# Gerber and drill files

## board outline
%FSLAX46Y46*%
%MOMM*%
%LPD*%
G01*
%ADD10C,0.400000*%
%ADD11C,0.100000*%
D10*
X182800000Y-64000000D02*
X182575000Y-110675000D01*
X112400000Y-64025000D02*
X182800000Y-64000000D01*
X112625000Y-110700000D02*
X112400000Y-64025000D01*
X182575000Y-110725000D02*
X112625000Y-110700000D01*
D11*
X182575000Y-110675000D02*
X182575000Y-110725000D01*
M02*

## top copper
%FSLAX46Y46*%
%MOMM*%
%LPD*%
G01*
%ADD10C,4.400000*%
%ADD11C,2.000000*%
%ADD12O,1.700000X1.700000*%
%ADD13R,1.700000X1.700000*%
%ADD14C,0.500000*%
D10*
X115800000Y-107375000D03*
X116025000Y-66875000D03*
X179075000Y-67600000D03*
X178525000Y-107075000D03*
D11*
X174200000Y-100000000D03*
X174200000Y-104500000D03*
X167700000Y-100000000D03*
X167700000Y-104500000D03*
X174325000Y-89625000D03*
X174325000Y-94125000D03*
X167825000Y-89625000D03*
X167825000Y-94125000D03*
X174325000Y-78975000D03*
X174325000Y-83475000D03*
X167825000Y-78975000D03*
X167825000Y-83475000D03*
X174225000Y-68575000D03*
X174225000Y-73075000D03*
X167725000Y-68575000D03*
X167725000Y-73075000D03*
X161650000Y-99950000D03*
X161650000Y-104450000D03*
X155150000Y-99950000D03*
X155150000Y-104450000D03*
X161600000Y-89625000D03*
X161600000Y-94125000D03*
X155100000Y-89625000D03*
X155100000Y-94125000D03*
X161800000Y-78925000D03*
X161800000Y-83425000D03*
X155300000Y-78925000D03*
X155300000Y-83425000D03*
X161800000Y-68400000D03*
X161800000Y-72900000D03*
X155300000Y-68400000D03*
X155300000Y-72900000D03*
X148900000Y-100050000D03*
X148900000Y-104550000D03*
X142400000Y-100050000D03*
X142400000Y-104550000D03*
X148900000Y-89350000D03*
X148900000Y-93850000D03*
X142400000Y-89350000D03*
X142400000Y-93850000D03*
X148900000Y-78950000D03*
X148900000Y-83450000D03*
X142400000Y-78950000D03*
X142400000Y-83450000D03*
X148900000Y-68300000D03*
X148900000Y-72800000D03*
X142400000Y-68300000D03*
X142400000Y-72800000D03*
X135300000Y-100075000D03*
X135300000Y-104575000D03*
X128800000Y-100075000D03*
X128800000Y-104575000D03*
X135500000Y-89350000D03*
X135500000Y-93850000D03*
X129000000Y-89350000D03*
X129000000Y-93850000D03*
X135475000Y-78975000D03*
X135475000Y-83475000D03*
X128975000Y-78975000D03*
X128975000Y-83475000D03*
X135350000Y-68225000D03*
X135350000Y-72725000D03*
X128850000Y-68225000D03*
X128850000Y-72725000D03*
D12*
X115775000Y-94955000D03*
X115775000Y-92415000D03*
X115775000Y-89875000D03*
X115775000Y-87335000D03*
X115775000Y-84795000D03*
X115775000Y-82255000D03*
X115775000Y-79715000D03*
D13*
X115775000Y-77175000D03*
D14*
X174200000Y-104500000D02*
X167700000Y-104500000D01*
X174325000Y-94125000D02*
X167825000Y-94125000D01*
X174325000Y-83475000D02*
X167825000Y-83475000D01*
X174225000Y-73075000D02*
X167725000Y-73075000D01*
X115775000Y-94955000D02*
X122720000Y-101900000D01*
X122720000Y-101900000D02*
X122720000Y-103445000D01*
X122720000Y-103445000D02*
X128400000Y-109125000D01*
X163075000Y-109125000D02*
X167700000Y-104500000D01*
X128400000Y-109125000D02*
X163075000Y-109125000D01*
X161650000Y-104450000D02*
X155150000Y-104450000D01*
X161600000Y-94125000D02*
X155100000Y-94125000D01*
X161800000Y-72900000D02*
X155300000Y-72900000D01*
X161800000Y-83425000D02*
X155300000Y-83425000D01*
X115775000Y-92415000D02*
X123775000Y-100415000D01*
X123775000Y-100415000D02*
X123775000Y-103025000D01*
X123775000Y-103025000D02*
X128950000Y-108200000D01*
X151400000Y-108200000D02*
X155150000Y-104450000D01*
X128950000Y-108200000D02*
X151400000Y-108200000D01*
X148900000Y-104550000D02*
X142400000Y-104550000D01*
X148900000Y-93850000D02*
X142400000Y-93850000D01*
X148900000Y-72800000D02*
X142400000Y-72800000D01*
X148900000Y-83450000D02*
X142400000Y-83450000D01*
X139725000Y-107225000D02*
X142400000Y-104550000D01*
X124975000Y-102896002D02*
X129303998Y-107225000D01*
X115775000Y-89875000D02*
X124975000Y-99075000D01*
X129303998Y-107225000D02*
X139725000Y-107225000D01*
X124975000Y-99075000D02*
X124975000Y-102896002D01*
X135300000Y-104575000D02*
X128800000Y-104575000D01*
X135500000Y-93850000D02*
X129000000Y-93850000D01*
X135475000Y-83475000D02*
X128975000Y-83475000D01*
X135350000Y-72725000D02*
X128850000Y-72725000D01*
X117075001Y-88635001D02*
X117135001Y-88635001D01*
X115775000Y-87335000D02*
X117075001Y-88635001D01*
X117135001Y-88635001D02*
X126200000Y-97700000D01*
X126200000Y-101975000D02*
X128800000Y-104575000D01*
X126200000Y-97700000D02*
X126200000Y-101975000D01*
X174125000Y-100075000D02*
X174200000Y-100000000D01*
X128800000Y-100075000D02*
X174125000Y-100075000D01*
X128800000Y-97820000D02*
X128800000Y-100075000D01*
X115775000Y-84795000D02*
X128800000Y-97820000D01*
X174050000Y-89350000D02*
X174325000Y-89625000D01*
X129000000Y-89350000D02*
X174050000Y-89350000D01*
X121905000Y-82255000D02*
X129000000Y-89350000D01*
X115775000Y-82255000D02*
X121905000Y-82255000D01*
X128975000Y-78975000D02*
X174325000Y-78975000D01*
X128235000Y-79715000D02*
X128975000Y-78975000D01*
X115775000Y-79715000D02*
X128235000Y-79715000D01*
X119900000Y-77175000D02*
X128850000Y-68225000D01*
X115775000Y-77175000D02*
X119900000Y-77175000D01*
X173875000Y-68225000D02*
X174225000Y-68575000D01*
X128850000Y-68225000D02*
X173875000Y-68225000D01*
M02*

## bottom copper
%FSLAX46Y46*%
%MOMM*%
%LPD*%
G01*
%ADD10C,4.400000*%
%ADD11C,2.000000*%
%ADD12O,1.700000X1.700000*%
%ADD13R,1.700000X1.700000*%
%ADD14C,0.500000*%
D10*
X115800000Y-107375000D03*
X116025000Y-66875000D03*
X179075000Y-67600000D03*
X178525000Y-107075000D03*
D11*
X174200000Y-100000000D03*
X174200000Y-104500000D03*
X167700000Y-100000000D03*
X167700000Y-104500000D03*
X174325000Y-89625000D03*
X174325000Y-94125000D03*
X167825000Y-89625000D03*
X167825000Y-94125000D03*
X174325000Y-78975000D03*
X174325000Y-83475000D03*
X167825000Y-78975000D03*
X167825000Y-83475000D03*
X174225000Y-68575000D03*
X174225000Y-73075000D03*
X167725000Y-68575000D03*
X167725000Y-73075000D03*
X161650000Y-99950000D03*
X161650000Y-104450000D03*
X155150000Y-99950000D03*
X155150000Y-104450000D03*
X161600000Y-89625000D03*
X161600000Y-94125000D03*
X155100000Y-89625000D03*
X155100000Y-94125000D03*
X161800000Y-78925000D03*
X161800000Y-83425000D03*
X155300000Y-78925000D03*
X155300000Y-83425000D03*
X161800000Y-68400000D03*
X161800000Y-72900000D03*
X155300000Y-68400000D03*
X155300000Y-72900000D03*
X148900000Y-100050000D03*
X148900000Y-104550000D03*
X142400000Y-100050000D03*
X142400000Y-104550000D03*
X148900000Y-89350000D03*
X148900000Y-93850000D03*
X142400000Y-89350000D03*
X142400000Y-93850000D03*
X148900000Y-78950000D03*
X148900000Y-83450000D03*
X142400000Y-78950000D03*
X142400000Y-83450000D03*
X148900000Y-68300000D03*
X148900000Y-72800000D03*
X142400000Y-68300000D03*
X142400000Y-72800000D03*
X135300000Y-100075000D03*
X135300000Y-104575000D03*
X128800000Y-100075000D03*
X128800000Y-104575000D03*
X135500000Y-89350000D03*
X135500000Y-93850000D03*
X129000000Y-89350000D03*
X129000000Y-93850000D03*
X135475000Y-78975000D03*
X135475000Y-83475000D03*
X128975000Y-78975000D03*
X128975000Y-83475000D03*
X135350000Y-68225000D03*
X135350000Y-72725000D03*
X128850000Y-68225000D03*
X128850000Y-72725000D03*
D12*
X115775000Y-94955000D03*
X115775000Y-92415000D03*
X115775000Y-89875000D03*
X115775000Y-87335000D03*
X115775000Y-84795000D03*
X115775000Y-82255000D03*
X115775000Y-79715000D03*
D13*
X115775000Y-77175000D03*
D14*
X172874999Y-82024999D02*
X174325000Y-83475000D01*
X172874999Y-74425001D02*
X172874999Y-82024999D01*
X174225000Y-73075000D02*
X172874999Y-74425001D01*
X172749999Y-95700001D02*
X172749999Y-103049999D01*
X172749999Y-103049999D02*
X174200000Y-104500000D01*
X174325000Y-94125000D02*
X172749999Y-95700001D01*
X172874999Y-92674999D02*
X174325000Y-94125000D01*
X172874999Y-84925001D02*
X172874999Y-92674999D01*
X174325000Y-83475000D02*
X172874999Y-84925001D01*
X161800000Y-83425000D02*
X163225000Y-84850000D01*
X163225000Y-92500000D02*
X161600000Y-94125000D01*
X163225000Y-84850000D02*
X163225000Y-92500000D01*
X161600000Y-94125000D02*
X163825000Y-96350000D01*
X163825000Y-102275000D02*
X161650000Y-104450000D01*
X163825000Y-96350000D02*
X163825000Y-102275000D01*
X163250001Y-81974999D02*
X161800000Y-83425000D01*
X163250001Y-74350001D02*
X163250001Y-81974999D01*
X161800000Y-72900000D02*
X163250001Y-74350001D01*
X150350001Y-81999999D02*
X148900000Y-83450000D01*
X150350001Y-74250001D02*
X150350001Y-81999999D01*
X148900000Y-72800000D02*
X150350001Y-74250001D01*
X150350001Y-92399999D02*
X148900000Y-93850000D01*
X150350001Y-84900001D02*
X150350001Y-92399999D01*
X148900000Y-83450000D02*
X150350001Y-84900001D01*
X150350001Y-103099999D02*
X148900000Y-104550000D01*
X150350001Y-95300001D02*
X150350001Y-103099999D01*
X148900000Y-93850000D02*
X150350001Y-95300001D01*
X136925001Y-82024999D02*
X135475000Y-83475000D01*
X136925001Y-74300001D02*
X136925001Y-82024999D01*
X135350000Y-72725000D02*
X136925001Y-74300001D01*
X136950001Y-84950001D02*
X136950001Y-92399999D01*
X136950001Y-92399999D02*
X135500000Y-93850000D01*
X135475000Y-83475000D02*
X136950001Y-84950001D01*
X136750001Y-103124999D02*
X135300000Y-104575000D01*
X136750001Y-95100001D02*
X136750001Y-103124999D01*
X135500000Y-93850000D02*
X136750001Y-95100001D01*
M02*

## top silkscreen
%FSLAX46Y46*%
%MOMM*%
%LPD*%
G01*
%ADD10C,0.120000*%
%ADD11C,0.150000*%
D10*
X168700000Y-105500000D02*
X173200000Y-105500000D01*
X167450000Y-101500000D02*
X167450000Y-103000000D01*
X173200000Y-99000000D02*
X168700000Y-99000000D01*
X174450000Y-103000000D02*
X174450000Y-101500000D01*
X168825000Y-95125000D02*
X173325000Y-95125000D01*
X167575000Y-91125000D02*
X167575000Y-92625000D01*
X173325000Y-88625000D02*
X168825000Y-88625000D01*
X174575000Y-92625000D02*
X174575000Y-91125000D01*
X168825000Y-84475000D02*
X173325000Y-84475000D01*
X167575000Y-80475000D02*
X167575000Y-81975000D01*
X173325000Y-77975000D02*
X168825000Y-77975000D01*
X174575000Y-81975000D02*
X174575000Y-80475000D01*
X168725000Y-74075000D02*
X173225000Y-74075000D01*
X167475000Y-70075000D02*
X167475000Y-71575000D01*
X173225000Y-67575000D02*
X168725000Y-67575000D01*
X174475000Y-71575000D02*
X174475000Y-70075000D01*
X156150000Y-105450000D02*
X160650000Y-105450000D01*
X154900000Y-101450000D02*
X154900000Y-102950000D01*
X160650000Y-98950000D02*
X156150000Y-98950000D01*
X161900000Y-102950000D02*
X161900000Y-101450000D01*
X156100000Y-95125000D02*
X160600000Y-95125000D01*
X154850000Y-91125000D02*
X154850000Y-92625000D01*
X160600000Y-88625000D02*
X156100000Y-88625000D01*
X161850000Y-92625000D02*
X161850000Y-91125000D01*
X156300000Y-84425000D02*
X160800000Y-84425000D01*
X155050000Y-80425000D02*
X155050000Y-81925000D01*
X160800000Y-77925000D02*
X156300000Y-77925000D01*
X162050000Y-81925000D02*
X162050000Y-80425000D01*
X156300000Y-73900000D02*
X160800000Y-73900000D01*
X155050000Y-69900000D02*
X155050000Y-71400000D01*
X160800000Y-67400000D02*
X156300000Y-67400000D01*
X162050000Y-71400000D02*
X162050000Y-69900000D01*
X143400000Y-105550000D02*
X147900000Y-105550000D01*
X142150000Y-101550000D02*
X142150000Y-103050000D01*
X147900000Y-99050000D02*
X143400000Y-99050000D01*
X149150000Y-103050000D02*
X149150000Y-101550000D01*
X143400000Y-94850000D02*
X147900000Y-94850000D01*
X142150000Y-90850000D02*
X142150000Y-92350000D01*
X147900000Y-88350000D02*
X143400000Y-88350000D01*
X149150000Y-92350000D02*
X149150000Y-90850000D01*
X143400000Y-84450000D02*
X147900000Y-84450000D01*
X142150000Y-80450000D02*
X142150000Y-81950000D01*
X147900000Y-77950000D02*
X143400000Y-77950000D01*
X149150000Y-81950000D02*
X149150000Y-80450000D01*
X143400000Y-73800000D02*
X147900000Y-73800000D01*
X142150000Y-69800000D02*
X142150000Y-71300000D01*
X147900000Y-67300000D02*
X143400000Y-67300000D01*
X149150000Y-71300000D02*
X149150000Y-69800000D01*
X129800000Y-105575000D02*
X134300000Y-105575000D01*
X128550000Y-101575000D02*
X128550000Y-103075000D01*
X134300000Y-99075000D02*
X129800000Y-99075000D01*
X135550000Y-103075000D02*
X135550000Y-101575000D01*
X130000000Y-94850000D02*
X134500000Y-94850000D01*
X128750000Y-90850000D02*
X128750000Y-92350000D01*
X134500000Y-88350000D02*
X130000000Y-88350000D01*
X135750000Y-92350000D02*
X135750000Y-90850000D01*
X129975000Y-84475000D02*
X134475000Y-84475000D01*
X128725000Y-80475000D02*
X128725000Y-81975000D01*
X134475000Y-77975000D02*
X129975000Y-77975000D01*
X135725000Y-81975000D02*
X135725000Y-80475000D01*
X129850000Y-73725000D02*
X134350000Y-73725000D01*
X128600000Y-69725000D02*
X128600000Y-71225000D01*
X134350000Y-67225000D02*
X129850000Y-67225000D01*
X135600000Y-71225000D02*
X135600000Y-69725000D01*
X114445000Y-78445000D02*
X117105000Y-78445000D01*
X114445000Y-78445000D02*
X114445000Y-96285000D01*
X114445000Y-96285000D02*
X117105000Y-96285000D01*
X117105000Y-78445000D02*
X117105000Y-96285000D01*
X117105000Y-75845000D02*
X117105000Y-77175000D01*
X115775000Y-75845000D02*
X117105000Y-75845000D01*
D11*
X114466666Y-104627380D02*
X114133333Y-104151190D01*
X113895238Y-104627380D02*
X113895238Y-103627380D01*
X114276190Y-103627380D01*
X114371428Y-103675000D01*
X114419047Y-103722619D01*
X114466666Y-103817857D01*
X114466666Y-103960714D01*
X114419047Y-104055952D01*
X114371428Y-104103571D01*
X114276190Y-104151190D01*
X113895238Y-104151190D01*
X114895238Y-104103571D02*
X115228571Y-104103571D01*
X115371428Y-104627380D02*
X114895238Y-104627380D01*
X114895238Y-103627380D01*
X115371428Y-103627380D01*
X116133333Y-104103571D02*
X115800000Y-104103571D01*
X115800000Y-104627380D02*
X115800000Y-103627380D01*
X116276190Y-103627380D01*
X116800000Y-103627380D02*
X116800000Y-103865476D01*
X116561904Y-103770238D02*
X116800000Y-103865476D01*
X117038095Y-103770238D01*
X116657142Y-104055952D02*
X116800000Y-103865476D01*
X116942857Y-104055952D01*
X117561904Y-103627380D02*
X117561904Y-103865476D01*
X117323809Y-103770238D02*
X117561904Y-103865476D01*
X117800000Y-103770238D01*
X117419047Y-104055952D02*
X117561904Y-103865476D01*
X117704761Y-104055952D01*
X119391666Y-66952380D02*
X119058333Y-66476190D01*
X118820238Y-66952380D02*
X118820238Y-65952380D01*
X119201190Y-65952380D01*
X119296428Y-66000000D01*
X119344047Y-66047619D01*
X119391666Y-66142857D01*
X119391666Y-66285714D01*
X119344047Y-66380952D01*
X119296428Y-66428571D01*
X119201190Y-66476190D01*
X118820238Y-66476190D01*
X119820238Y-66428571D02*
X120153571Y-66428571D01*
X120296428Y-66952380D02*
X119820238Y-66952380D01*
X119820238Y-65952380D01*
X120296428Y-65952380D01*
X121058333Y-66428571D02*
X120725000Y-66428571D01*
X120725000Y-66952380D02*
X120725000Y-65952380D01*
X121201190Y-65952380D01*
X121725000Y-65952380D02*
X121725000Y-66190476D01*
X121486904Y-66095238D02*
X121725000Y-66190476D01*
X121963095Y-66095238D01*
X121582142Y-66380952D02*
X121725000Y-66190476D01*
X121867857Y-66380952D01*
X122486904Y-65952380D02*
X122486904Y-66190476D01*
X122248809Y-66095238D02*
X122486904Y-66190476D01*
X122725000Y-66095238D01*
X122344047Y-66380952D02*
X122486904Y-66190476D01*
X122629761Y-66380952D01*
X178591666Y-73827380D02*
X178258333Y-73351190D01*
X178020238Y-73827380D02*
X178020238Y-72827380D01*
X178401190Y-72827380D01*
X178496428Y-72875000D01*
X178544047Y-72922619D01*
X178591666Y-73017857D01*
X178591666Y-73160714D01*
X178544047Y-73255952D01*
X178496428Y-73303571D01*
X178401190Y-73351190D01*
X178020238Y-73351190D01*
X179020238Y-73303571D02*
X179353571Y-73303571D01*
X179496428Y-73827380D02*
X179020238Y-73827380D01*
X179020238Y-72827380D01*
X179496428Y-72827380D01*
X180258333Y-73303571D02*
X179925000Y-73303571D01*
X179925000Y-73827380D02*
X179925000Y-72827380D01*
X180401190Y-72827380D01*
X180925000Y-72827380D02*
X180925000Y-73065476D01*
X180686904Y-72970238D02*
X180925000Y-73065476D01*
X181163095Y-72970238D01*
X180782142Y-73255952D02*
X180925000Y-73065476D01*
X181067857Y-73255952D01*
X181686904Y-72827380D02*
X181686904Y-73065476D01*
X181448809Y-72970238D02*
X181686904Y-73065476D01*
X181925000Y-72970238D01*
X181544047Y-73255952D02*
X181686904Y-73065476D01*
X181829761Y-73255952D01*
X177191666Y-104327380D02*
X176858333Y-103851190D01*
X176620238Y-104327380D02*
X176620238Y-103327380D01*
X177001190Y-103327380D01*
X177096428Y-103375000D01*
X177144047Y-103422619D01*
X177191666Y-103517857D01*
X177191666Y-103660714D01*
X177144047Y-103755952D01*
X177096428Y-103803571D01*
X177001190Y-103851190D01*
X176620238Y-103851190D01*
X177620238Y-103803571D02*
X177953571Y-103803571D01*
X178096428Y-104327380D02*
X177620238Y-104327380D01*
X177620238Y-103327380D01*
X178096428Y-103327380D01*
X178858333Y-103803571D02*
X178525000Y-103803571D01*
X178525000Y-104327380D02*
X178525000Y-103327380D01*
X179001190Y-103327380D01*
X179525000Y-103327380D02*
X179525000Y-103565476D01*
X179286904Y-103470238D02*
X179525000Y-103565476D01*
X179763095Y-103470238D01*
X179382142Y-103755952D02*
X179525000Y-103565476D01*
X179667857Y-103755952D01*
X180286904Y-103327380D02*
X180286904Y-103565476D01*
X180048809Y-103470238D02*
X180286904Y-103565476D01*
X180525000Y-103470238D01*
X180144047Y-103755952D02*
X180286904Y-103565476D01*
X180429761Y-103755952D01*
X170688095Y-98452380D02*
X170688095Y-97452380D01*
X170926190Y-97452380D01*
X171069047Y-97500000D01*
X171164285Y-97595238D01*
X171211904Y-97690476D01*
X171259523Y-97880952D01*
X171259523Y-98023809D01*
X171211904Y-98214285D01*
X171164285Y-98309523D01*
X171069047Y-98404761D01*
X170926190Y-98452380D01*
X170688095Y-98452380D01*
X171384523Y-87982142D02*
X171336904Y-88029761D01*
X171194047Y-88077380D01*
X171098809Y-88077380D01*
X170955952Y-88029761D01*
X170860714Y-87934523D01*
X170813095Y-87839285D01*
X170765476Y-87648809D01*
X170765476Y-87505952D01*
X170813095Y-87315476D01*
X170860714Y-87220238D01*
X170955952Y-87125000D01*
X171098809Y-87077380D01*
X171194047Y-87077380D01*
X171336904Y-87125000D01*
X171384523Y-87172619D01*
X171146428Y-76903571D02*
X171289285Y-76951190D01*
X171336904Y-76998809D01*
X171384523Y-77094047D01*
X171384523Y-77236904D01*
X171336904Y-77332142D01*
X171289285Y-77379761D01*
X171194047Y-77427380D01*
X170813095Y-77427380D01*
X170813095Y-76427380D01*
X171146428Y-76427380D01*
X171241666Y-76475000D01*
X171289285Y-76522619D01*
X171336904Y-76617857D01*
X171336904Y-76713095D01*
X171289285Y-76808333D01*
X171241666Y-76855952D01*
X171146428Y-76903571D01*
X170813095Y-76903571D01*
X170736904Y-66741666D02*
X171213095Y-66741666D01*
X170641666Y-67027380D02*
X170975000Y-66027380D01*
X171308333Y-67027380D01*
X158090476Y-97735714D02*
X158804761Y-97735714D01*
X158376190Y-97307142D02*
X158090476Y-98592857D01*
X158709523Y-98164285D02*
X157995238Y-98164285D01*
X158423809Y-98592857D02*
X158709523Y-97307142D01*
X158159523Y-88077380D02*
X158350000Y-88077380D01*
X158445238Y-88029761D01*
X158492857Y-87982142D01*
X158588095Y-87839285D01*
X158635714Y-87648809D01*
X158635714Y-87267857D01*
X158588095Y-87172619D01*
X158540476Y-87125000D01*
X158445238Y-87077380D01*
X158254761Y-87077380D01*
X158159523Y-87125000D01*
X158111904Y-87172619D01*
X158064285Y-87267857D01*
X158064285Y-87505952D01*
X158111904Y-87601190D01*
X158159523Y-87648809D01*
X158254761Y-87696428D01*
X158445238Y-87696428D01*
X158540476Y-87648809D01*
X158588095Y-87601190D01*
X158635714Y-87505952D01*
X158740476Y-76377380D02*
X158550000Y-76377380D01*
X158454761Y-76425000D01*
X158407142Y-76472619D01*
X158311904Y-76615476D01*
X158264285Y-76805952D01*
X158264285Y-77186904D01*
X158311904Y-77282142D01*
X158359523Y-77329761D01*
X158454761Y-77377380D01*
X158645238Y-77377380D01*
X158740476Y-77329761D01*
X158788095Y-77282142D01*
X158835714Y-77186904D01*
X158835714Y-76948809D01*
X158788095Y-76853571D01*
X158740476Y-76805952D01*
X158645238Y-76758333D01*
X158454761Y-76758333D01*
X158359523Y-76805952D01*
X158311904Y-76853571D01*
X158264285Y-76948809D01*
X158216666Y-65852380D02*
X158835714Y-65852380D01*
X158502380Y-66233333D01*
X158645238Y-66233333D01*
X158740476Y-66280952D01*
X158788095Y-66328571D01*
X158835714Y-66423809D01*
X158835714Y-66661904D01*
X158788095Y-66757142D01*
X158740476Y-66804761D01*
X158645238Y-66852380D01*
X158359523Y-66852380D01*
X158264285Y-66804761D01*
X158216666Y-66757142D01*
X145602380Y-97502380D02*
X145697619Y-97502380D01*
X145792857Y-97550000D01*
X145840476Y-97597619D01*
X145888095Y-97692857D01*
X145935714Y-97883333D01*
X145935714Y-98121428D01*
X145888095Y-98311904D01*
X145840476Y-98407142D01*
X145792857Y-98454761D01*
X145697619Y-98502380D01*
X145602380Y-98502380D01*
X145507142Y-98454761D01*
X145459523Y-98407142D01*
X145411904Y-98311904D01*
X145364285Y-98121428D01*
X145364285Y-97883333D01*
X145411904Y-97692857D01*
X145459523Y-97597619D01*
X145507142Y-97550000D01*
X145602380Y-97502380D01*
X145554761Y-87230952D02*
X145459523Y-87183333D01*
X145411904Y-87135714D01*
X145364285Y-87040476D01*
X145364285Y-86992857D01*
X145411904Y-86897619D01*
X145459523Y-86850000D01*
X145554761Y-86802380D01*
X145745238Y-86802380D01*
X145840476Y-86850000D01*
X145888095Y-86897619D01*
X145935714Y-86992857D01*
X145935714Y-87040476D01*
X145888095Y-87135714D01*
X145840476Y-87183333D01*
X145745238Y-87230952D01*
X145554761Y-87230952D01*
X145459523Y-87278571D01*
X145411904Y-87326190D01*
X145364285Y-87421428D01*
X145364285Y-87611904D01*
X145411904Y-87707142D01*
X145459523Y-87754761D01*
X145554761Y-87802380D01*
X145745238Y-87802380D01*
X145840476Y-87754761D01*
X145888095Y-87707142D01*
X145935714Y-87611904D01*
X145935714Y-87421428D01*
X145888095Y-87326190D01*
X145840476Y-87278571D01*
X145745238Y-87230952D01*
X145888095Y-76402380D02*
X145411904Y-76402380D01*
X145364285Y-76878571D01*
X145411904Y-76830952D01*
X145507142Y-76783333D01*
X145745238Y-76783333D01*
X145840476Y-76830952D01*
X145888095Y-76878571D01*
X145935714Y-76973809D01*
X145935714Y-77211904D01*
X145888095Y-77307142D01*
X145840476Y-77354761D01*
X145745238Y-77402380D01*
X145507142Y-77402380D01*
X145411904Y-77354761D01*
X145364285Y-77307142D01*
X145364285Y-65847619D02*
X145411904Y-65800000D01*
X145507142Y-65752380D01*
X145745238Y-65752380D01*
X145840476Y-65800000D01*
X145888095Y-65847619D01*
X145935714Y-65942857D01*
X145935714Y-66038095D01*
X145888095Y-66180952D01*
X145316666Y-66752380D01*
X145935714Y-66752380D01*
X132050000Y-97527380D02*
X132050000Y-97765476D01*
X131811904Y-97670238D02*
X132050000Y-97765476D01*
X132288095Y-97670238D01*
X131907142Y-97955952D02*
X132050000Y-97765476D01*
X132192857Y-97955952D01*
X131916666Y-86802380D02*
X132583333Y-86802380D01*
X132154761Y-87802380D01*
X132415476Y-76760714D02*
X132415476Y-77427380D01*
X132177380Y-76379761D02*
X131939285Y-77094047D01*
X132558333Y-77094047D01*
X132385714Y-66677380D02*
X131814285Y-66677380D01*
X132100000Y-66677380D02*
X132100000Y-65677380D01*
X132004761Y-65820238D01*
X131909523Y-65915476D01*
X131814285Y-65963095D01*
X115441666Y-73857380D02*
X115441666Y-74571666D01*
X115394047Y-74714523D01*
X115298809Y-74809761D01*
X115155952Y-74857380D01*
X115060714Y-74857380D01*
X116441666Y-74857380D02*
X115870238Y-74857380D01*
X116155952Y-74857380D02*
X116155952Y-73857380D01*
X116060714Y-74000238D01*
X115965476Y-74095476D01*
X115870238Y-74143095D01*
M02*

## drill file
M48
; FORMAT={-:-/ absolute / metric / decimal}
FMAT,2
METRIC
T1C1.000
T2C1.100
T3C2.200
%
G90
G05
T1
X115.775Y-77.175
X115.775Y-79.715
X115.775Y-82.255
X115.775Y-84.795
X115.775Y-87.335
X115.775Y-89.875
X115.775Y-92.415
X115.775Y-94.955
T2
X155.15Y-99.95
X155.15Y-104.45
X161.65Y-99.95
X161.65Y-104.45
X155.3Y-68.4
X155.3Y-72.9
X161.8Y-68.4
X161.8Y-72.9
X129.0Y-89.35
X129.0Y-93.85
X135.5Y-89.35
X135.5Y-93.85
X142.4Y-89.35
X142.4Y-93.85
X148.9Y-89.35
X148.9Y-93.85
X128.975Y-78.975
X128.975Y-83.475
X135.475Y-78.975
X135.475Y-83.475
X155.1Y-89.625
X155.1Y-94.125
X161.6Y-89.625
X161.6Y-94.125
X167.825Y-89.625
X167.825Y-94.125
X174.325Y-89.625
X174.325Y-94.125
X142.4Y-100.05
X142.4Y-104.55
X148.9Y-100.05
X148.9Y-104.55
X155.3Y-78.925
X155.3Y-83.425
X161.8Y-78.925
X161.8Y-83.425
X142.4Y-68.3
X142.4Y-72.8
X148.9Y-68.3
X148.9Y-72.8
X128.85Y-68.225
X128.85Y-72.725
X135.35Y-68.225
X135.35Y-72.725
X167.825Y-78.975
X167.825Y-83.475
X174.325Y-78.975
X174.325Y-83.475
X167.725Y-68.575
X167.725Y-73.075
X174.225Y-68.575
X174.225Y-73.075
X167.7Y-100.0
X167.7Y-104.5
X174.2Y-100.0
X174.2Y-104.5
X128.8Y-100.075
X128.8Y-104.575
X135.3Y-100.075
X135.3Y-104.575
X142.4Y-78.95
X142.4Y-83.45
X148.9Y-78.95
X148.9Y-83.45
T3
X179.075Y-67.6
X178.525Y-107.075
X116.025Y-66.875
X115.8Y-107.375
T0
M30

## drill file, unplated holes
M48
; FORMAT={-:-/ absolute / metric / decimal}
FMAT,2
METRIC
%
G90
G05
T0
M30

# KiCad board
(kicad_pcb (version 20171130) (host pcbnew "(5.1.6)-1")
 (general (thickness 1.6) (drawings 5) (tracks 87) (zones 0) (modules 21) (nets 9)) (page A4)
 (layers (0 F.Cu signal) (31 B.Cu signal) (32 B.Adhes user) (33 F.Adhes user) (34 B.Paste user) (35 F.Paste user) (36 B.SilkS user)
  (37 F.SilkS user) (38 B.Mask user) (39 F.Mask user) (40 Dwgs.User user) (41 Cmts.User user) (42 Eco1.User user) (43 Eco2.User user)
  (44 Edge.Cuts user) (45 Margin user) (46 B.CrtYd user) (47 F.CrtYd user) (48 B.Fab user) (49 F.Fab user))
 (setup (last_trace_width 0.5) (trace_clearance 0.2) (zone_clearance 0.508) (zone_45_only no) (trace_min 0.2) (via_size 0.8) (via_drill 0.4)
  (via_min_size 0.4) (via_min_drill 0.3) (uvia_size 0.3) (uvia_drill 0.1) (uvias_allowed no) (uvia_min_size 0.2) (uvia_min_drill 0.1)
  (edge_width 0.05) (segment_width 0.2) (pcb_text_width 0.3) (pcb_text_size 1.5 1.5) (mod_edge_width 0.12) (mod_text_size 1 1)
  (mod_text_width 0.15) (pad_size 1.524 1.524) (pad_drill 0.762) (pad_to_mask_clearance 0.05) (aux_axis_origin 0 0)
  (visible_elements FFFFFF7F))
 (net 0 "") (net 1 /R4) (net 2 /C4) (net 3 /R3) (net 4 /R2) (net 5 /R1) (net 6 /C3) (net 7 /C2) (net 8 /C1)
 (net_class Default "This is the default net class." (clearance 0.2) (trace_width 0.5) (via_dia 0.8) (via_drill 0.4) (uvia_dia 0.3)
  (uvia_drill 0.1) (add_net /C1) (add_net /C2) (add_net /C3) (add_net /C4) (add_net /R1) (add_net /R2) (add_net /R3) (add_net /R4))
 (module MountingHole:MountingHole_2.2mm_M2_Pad (layer F.Cu) (at 115.8 107.375)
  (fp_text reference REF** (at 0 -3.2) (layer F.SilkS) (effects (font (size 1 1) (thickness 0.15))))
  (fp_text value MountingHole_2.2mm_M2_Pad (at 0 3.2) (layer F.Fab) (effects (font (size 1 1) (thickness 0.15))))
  (pad 1 thru_hole circle (at 0 0) (size 4.4 4.4) (drill 2.2) (layers *.Cu *.Mask)))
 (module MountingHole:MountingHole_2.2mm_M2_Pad (layer F.Cu) (at 116.025 66.875)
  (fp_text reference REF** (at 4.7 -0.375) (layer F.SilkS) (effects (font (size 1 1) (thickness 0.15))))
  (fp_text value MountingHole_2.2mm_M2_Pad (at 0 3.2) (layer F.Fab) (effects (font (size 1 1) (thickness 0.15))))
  (pad 1 thru_hole circle (at 0 0) (size 4.4 4.4) (drill 2.2) (layers *.Cu *.Mask)))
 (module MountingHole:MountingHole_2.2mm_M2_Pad (layer F.Cu) (at 179.075 67.6)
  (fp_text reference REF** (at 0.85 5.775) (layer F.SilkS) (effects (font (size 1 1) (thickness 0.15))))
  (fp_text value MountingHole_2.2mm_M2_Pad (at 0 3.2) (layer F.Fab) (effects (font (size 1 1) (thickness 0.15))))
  (pad 1 thru_hole circle (at 0 0) (size 4.4 4.4) (drill 2.2) (layers *.Cu *.Mask)))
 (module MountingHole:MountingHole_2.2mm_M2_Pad (layer F.Cu) (at 178.525 107.075)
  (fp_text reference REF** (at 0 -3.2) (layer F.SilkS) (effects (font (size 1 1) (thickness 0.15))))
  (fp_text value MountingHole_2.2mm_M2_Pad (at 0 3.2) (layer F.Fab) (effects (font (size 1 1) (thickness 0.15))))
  (pad 1 thru_hole circle (at 0 0) (size 4.4 4.4) (drill 2.2) (layers *.Cu *.Mask)))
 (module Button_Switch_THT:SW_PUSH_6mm (layer F.Cu) (at 167.7 100)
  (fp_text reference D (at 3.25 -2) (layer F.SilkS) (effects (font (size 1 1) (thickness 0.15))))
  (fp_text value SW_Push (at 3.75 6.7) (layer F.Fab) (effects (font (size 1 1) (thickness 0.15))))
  (fp_line (start 1 5.5) (end 5.5 5.5) (layer F.SilkS) (width 0.12))
  (fp_line (start -0.25 1.5) (end -0.25 3) (layer F.SilkS) (width 0.12))
  (fp_line (start 5.5 -1) (end 1 -1) (layer F.SilkS) (width 0.12))
  (fp_line (start 6.75 3) (end 6.75 1.5) (layer F.SilkS) (width 0.12))
  (pad 1 thru_hole circle (at 6.5 0 90) (size 2 2) (drill 1.1) (layers *.Cu *.Mask) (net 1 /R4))
  (pad 2 thru_hole circle (at 6.5 4.5 90) (size 2 2) (drill 1.1) (layers *.Cu *.Mask) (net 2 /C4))
  (pad 1 thru_hole circle (at 0 0 90) (size 2 2) (drill 1.1) (layers *.Cu *.Mask) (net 1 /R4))
  (pad 2 thru_hole circle (at 0 4.5 90) (size 2 2) (drill 1.1) (layers *.Cu *.Mask) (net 2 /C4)))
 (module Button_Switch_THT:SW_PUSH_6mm (layer F.Cu) (at 167.825 89.625)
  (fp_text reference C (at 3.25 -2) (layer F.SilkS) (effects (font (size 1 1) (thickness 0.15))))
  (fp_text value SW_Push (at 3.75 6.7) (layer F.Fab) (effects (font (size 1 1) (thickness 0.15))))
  (fp_line (start 1 5.5) (end 5.5 5.5) (layer F.SilkS) (width 0.12))
  (fp_line (start -0.25 1.5) (end -0.25 3) (layer F.SilkS) (width 0.12))
  (fp_line (start 5.5 -1) (end 1 -1) (layer F.SilkS) (width 0.12))
  (fp_line (start 6.75 3) (end 6.75 1.5) (layer F.SilkS) (width 0.12))
  (pad 1 thru_hole circle (at 6.5 0 90) (size 2 2) (drill 1.1) (layers *.Cu *.Mask) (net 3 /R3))
  (pad 2 thru_hole circle (at 6.5 4.5 90) (size 2 2) (drill 1.1) (layers *.Cu *.Mask) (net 2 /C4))
  (pad 1 thru_hole circle (at 0 0 90) (size 2 2) (drill 1.1) (layers *.Cu *.Mask) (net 3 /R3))
  (pad 2 thru_hole circle (at 0 4.5 90) (size 2 2) (drill 1.1) (layers *.Cu *.Mask) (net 2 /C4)))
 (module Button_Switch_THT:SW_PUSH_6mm (layer F.Cu) (at 167.825 78.975)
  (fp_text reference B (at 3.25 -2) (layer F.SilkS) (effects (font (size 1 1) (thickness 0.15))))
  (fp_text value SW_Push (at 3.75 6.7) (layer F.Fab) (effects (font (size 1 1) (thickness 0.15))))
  (fp_line (start 1 5.5) (end 5.5 5.5) (layer F.SilkS) (width 0.12))
  (fp_line (start -0.25 1.5) (end -0.25 3) (layer F.SilkS) (width 0.12))
  (fp_line (start 5.5 -1) (end 1 -1) (layer F.SilkS) (width 0.12))
  (fp_line (start 6.75 3) (end 6.75 1.5) (layer F.SilkS) (width 0.12))
  (pad 1 thru_hole circle (at 6.5 0 90) (size 2 2) (drill 1.1) (layers *.Cu *.Mask) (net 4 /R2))
  (pad 2 thru_hole circle (at 6.5 4.5 90) (size 2 2) (drill 1.1) (layers *.Cu *.Mask) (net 2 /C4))
  (pad 1 thru_hole circle (at 0 0 90) (size 2 2) (drill 1.1) (layers *.Cu *.Mask) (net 4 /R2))
  (pad 2 thru_hole circle (at 0 4.5 90) (size 2 2) (drill 1.1) (layers *.Cu *.Mask) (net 2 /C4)))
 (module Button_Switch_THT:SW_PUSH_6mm (layer F.Cu) (at 167.725 68.575)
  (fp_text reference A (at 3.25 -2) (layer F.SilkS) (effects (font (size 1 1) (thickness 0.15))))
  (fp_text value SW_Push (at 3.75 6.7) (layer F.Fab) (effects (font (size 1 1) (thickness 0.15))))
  (fp_line (start 1 5.5) (end 5.5 5.5) (layer F.SilkS) (width 0.12))
  (fp_line (start -0.25 1.5) (end -0.25 3) (layer F.SilkS) (width 0.12))
  (fp_line (start 5.5 -1) (end 1 -1) (layer F.SilkS) (width 0.12))
  (fp_line (start 6.75 3) (end 6.75 1.5) (layer F.SilkS) (width 0.12))
  (pad 1 thru_hole circle (at 6.5 0 90) (size 2 2) (drill 1.1) (layers *.Cu *.Mask) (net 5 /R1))
  (pad 2 thru_hole circle (at 6.5 4.5 90) (size 2 2) (drill 1.1) (layers *.Cu *.Mask) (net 2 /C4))
  (pad 1 thru_hole circle (at 0 0 90) (size 2 2) (drill 1.1) (layers *.Cu *.Mask) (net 5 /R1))
  (pad 2 thru_hole circle (at 0 4.5 90) (size 2 2) (drill 1.1) (layers *.Cu *.Mask) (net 2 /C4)))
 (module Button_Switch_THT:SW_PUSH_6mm (layer F.Cu) (at 155.15 99.95)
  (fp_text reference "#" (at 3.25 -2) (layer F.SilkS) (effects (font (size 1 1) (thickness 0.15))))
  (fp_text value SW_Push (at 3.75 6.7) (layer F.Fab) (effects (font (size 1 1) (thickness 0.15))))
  (fp_line (start 1 5.5) (end 5.5 5.5) (layer F.SilkS) (width 0.12))
  (fp_line (start -0.25 1.5) (end -0.25 3) (layer F.SilkS) (width 0.12))
  (fp_line (start 5.5 -1) (end 1 -1) (layer F.SilkS) (width 0.12))
  (fp_line (start 6.75 3) (end 6.75 1.5) (layer F.SilkS) (width 0.12))
  (pad 1 thru_hole circle (at 6.5 0 90) (size 2 2) (drill 1.1) (layers *.Cu *.Mask) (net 1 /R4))
  (pad 2 thru_hole circle (at 6.5 4.5 90) (size 2 2) (drill 1.1) (layers *.Cu *.Mask) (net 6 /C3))
  (pad 1 thru_hole circle (at 0 0 90) (size 2 2) (drill 1.1) (layers *.Cu *.Mask) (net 1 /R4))
  (pad 2 thru_hole circle (at 0 4.5 90) (size 2 2) (drill 1.1) (layers *.Cu *.Mask) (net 6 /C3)))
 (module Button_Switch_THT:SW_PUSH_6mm (layer F.Cu) (at 155.1 89.625)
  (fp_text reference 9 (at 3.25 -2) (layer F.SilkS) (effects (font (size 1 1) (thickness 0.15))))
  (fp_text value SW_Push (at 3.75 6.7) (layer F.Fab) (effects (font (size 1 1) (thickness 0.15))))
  (fp_line (start 1 5.5) (end 5.5 5.5) (layer F.SilkS) (width 0.12))
  (fp_line (start -0.25 1.5) (end -0.25 3) (layer F.SilkS) (width 0.12))
  (fp_line (start 5.5 -1) (end 1 -1) (layer F.SilkS) (width 0.12))
  (fp_line (start 6.75 3) (end 6.75 1.5) (layer F.SilkS) (width 0.12))
  (pad 1 thru_hole circle (at 6.5 0 90) (size 2 2) (drill 1.1) (layers *.Cu *.Mask) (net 3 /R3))
  (pad 2 thru_hole circle (at 6.5 4.5 90) (size 2 2) (drill 1.1) (layers *.Cu *.Mask) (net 6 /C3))
  (pad 1 thru_hole circle (at 0 0 90) (size 2 2) (drill 1.1) (layers *.Cu *.Mask) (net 3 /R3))
  (pad 2 thru_hole circle (at 0 4.5 90) (size 2 2) (drill 1.1) (layers *.Cu *.Mask) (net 6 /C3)))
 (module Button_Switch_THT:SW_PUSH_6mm (layer F.Cu) (at 155.3 78.925)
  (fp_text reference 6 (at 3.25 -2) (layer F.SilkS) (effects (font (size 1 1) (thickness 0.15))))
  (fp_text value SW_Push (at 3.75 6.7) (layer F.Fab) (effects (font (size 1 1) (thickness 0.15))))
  (fp_line (start 1 5.5) (end 5.5 5.5) (layer F.SilkS) (width 0.12))
  (fp_line (start -0.25 1.5) (end -0.25 3) (layer F.SilkS) (width 0.12))
  (fp_line (start 5.5 -1) (end 1 -1) (layer F.SilkS) (width 0.12))
  (fp_line (start 6.75 3) (end 6.75 1.5) (layer F.SilkS) (width 0.12))
  (pad 1 thru_hole circle (at 6.5 0 90) (size 2 2) (drill 1.1) (layers *.Cu *.Mask) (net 4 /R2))
  (pad 2 thru_hole circle (at 6.5 4.5 90) (size 2 2) (drill 1.1) (layers *.Cu *.Mask) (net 6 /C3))
  (pad 1 thru_hole circle (at 0 0 90) (size 2 2) (drill 1.1) (layers *.Cu *.Mask) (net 4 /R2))
  (pad 2 thru_hole circle (at 0 4.5 90) (size 2 2) (drill 1.1) (layers *.Cu *.Mask) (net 6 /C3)))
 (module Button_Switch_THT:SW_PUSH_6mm (layer F.Cu) (at 155.3 68.4)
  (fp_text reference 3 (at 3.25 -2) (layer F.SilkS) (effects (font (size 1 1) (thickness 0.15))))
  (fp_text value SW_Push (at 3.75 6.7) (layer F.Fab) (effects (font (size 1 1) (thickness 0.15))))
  (fp_line (start 1 5.5) (end 5.5 5.5) (layer F.SilkS) (width 0.12))
  (fp_line (start -0.25 1.5) (end -0.25 3) (layer F.SilkS) (width 0.12))
  (fp_line (start 5.5 -1) (end 1 -1) (layer F.SilkS) (width 0.12))
  (fp_line (start 6.75 3) (end 6.75 1.5) (layer F.SilkS) (width 0.12))
  (pad 1 thru_hole circle (at 6.5 0 90) (size 2 2) (drill 1.1) (layers *.Cu *.Mask) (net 5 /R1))
  (pad 2 thru_hole circle (at 6.5 4.5 90) (size 2 2) (drill 1.1) (layers *.Cu *.Mask) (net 6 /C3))
  (pad 1 thru_hole circle (at 0 0 90) (size 2 2) (drill 1.1) (layers *.Cu *.Mask) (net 5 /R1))
  (pad 2 thru_hole circle (at 0 4.5 90) (size 2 2) (drill 1.1) (layers *.Cu *.Mask) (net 6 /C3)))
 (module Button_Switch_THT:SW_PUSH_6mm (layer F.Cu) (at 142.4 100.05)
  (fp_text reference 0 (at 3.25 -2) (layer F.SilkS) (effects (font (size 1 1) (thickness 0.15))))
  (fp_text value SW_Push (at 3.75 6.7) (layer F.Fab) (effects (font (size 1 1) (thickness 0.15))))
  (fp_line (start 1 5.5) (end 5.5 5.5) (layer F.SilkS) (width 0.12))
  (fp_line (start -0.25 1.5) (end -0.25 3) (layer F.SilkS) (width 0.12))
  (fp_line (start 5.5 -1) (end 1 -1) (layer F.SilkS) (width 0.12))
  (fp_line (start 6.75 3) (end 6.75 1.5) (layer F.SilkS) (width 0.12))
  (pad 1 thru_hole circle (at 6.5 0 90) (size 2 2) (drill 1.1) (layers *.Cu *.Mask) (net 1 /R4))
  (pad 2 thru_hole circle (at 6.5 4.5 90) (size 2 2) (drill 1.1) (layers *.Cu *.Mask) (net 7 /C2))
  (pad 1 thru_hole circle (at 0 0 90) (size 2 2) (drill 1.1) (layers *.Cu *.Mask) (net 1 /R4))
  (pad 2 thru_hole circle (at 0 4.5 90) (size 2 2) (drill 1.1) (layers *.Cu *.Mask) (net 7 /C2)))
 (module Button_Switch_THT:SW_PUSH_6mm (layer F.Cu) (at 142.4 89.35)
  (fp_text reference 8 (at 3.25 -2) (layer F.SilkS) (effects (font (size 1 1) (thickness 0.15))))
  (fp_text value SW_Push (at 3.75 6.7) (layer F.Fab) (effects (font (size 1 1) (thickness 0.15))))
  (fp_line (start 1 5.5) (end 5.5 5.5) (layer F.SilkS) (width 0.12))
  (fp_line (start -0.25 1.5) (end -0.25 3) (layer F.SilkS) (width 0.12))
  (fp_line (start 5.5 -1) (end 1 -1) (layer F.SilkS) (width 0.12))
  (fp_line (start 6.75 3) (end 6.75 1.5) (layer F.SilkS) (width 0.12))
  (pad 1 thru_hole circle (at 6.5 0 90) (size 2 2) (drill 1.1) (layers *.Cu *.Mask) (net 3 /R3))
  (pad 2 thru_hole circle (at 6.5 4.5 90) (size 2 2) (drill 1.1) (layers *.Cu *.Mask) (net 7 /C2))
  (pad 1 thru_hole circle (at 0 0 90) (size 2 2) (drill 1.1) (layers *.Cu *.Mask) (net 3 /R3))
  (pad 2 thru_hole circle (at 0 4.5 90) (size 2 2) (drill 1.1) (layers *.Cu *.Mask) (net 7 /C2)))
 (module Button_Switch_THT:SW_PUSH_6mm (layer F.Cu) (at 142.4 78.95)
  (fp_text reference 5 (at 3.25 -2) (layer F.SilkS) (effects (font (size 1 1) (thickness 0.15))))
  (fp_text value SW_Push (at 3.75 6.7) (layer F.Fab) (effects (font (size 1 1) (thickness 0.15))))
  (fp_line (start 1 5.5) (end 5.5 5.5) (layer F.SilkS) (width 0.12))
  (fp_line (start -0.25 1.5) (end -0.25 3) (layer F.SilkS) (width 0.12))
  (fp_line (start 5.5 -1) (end 1 -1) (layer F.SilkS) (width 0.12))
  (fp_line (start 6.75 3) (end 6.75 1.5) (layer F.SilkS) (width 0.12))
  (pad 1 thru_hole circle (at 6.5 0 90) (size 2 2) (drill 1.1) (layers *.Cu *.Mask) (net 4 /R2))
  (pad 2 thru_hole circle (at 6.5 4.5 90) (size 2 2) (drill 1.1) (layers *.Cu *.Mask) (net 7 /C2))
  (pad 1 thru_hole circle (at 0 0 90) (size 2 2) (drill 1.1) (layers *.Cu *.Mask) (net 4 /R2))
  (pad 2 thru_hole circle (at 0 4.5 90) (size 2 2) (drill 1.1) (layers *.Cu *.Mask) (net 7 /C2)))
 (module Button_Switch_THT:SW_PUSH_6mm (layer F.Cu) (at 142.4 68.3)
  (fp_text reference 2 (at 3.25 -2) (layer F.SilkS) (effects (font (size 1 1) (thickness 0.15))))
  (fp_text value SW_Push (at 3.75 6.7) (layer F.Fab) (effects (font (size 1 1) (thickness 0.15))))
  (fp_line (start 1 5.5) (end 5.5 5.5) (layer F.SilkS) (width 0.12))
  (fp_line (start -0.25 1.5) (end -0.25 3) (layer F.SilkS) (width 0.12))
  (fp_line (start 5.5 -1) (end 1 -1) (layer F.SilkS) (width 0.12))
  (fp_line (start 6.75 3) (end 6.75 1.5) (layer F.SilkS) (width 0.12))
  (pad 1 thru_hole circle (at 6.5 0 90) (size 2 2) (drill 1.1) (layers *.Cu *.Mask) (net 5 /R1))
  (pad 2 thru_hole circle (at 6.5 4.5 90) (size 2 2) (drill 1.1) (layers *.Cu *.Mask) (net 7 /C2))
  (pad 1 thru_hole circle (at 0 0 90) (size 2 2) (drill 1.1) (layers *.Cu *.Mask) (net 5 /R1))
  (pad 2 thru_hole circle (at 0 4.5 90) (size 2 2) (drill 1.1) (layers *.Cu *.Mask) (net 7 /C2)))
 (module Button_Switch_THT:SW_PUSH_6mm (layer F.Cu) (at 128.8 100.075)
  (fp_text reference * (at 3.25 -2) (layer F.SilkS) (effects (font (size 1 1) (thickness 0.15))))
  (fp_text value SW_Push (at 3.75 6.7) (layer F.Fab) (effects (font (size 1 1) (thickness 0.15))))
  (fp_line (start 1 5.5) (end 5.5 5.5) (layer F.SilkS) (width 0.12))
  (fp_line (start -0.25 1.5) (end -0.25 3) (layer F.SilkS) (width 0.12))
  (fp_line (start 5.5 -1) (end 1 -1) (layer F.SilkS) (width 0.12))
  (fp_line (start 6.75 3) (end 6.75 1.5) (layer F.SilkS) (width 0.12))
  (pad 1 thru_hole circle (at 6.5 0 90) (size 2 2) (drill 1.1) (layers *.Cu *.Mask) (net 1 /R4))
  (pad 2 thru_hole circle (at 6.5 4.5 90) (size 2 2) (drill 1.1) (layers *.Cu *.Mask) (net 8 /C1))
  (pad 1 thru_hole circle (at 0 0 90) (size 2 2) (drill 1.1) (layers *.Cu *.Mask) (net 1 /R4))
  (pad 2 thru_hole circle (at 0 4.5 90) (size 2 2) (drill 1.1) (layers *.Cu *.Mask) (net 8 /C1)))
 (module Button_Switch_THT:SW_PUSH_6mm (layer F.Cu) (at 129 89.35)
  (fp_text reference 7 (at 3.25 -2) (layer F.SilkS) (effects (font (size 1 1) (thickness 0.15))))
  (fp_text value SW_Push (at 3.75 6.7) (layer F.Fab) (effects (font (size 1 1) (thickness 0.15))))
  (fp_line (start 1 5.5) (end 5.5 5.5) (layer F.SilkS) (width 0.12))
  (fp_line (start -0.25 1.5) (end -0.25 3) (layer F.SilkS) (width 0.12))
  (fp_line (start 5.5 -1) (end 1 -1) (layer F.SilkS) (width 0.12))
  (fp_line (start 6.75 3) (end 6.75 1.5) (layer F.SilkS) (width 0.12))
  (pad 1 thru_hole circle (at 6.5 0 90) (size 2 2) (drill 1.1) (layers *.Cu *.Mask) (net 3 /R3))
  (pad 2 thru_hole circle (at 6.5 4.5 90) (size 2 2) (drill 1.1) (layers *.Cu *.Mask) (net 8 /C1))
  (pad 1 thru_hole circle (at 0 0 90) (size 2 2) (drill 1.1) (layers *.Cu *.Mask) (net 3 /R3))
  (pad 2 thru_hole circle (at 0 4.5 90) (size 2 2) (drill 1.1) (layers *.Cu *.Mask) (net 8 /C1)))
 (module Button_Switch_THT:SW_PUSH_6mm (layer F.Cu) (at 128.975 78.975)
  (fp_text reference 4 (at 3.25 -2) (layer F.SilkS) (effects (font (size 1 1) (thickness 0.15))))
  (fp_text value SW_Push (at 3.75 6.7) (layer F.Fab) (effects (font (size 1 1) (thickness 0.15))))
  (fp_line (start 1 5.5) (end 5.5 5.5) (layer F.SilkS) (width 0.12))
  (fp_line (start -0.25 1.5) (end -0.25 3) (layer F.SilkS) (width 0.12))
  (fp_line (start 5.5 -1) (end 1 -1) (layer F.SilkS) (width 0.12))
  (fp_line (start 6.75 3) (end 6.75 1.5) (layer F.SilkS) (width 0.12))
  (pad 1 thru_hole circle (at 6.5 0 90) (size 2 2) (drill 1.1) (layers *.Cu *.Mask) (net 4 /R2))
  (pad 2 thru_hole circle (at 6.5 4.5 90) (size 2 2) (drill 1.1) (layers *.Cu *.Mask) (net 8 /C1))
  (pad 1 thru_hole circle (at 0 0 90) (size 2 2) (drill 1.1) (layers *.Cu *.Mask) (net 4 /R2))
  (pad 2 thru_hole circle (at 0 4.5 90) (size 2 2) (drill 1.1) (layers *.Cu *.Mask) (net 8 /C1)))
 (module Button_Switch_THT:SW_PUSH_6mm (layer F.Cu) (at 128.85 68.225)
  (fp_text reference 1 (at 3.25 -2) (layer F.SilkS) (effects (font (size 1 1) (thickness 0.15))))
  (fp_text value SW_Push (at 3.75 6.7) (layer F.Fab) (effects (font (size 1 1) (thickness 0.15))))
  (fp_line (start 1 5.5) (end 5.5 5.5) (layer F.SilkS) (width 0.12))
  (fp_line (start -0.25 1.5) (end -0.25 3) (layer F.SilkS) (width 0.12))
  (fp_line (start 5.5 -1) (end 1 -1) (layer F.SilkS) (width 0.12))
  (fp_line (start 6.75 3) (end 6.75 1.5) (layer F.SilkS) (width 0.12))
  (pad 1 thru_hole circle (at 6.5 0 90) (size 2 2) (drill 1.1) (layers *.Cu *.Mask) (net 5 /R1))
  (pad 2 thru_hole circle (at 6.5 4.5 90) (size 2 2) (drill 1.1) (layers *.Cu *.Mask) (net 8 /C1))
  (pad 1 thru_hole circle (at 0 0 90) (size 2 2) (drill 1.1) (layers *.Cu *.Mask) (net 5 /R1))
  (pad 2 thru_hole circle (at 0 4.5 90) (size 2 2) (drill 1.1) (layers *.Cu *.Mask) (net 8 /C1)))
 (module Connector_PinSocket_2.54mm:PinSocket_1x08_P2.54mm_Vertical (layer F.Cu) (at 115.775 77.175)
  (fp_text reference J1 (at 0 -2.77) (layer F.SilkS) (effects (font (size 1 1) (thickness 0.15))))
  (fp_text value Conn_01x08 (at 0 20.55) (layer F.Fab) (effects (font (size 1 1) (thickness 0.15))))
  (fp_line (start -1.33 1.27) (end 1.33 1.27) (layer F.SilkS) (width 0.12))
  (fp_line (start -1.33 1.27) (end -1.33 19.11) (layer F.SilkS) (width 0.12))
  (fp_line (start -1.33 19.11) (end 1.33 19.11) (layer F.SilkS) (width 0.12))
  (fp_line (start 1.33 1.27) (end 1.33 19.11) (layer F.SilkS) (width 0.12))
  (fp_line (start 1.33 -1.33) (end 1.33 0) (layer F.SilkS) (width 0.12))
  (fp_line (start 0 -1.33) (end 1.33 -1.33) (layer F.SilkS) (width 0.12))
  (pad 8 thru_hole oval (at 0 17.78) (size 1.7 1.7) (drill 1) (layers *.Cu *.Mask) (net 2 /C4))
  (pad 7 thru_hole oval (at 0 15.24) (size 1.7 1.7) (drill 1) (layers *.Cu *.Mask) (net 6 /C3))
  (pad 6 thru_hole oval (at 0 12.7) (size 1.7 1.7) (drill 1) (layers *.Cu *.Mask) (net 7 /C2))
  (pad 5 thru_hole oval (at 0 10.16) (size 1.7 1.7) (drill 1) (layers *.Cu *.Mask) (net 8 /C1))
  (pad 4 thru_hole oval (at 0 7.62) (size 1.7 1.7) (drill 1) (layers *.Cu *.Mask) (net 1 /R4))
  (pad 3 thru_hole oval (at 0 5.08) (size 1.7 1.7) (drill 1) (layers *.Cu *.Mask) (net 3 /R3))
  (pad 2 thru_hole oval (at 0 2.54) (size 1.7 1.7) (drill 1) (layers *.Cu *.Mask) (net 4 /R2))
  (pad 1 thru_hole rect (at 0 0) (size 1.7 1.7) (drill 1) (layers *.Cu *.Mask) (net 5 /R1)))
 (gr_line (start 182.8 64) (end 182.575 110.675) (layer Edge.Cuts) (width 0.4))
 (gr_line (start 112.4 64.025) (end 182.8 64) (layer Edge.Cuts) (width 0.4))
 (gr_line (start 112.625 110.7) (end 112.4 64.025) (layer Edge.Cuts) (width 0.4))
 (gr_line (start 182.575 110.725) (end 112.625 110.7) (layer Edge.Cuts) (width 0.4))
 (gr_line (start 182.575 110.675) (end 182.575 110.725) (layer Edge.Cuts) (width 0.1))
 (segment (start 174.2 104.5) (end 167.7 104.5) (width 0.5) (layer F.Cu) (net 2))
 (segment (start 174.325 94.125) (end 167.825 94.125) (width 0.5) (layer F.Cu) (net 2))
 (segment (start 174.325 83.475) (end 167.825 83.475) (width 0.5) (layer F.Cu) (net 2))
 (segment (start 174.225 73.075) (end 167.725 73.075) (width 0.5) (layer F.Cu) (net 2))
 (segment (start 115.775 94.955) (end 122.72 101.9) (width 0.5) (layer F.Cu) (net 2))
 (segment (start 122.72 101.9) (end 122.72 103.445) (width 0.5) (layer F.Cu) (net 2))
 (segment (start 122.72 103.445) (end 128.4 109.125) (width 0.5) (layer F.Cu) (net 2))
 (segment (start 163.075 109.125) (end 167.7 104.5) (width 0.5) (layer F.Cu) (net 2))
 (segment (start 128.4 109.125) (end 163.075 109.125) (width 0.5) (layer F.Cu) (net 2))
 (segment (start 172.874999 82.024999) (end 174.325 83.475) (width 0.5) (layer B.Cu) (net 2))
 (segment (start 172.874999 74.425001) (end 172.874999 82.024999) (width 0.5) (layer B.Cu) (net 2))
 (segment (start 174.225 73.075) (end 172.874999 74.425001) (width 0.5) (layer B.Cu) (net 2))
 (segment (start 172.749999 95.700001) (end 172.749999 103.049999) (width 0.5) (layer B.Cu) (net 2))
 (segment (start 172.749999 103.049999) (end 174.2 104.5) (width 0.5) (layer B.Cu) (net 2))
 (segment (start 174.325 94.125) (end 172.749999 95.700001) (width 0.5) (layer B.Cu) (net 2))
 (segment (start 172.874999 92.674999) (end 174.325 94.125) (width 0.5) (layer B.Cu) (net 2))
 (segment (start 172.874999 84.925001) (end 172.874999 92.674999) (width 0.5) (layer B.Cu) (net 2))
 (segment (start 174.325 83.475) (end 172.874999 84.925001) (width 0.5) (layer B.Cu) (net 2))
 (segment (start 161.65 104.45) (end 155.15 104.45) (width 0.5) (layer F.Cu) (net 6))
 (segment (start 161.6 94.125) (end 155.1 94.125) (width 0.5) (layer F.Cu) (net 6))
 (segment (start 161.8 72.9) (end 155.3 72.9) (width 0.5) (layer F.Cu) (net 6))
 (segment (start 161.8 83.425) (end 155.3 83.425) (width 0.5) (layer F.Cu) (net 6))
 (segment (start 115.775 92.415) (end 123.775 100.415) (width 0.5) (layer F.Cu) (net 6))
 (segment (start 123.775 100.415) (end 123.775 103.025) (width 0.5) (layer F.Cu) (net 6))
 (segment (start 123.775 103.025) (end 128.95 108.2) (width 0.5) (layer F.Cu) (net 6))
 (segment (start 151.4 108.2) (end 155.15 104.45) (width 0.5) (layer F.Cu) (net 6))
 (segment (start 128.95 108.2) (end 151.4 108.2) (width 0.5) (layer F.Cu) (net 6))
 (segment (start 161.8 83.425) (end 163.225 84.85) (width 0.5) (layer B.Cu) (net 6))
 (segment (start 163.225 92.5) (end 161.6 94.125) (width 0.5) (layer B.Cu) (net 6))
 (segment (start 163.225 84.85) (end 163.225 92.5) (width 0.5) (layer B.Cu) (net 6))
 (segment (start 161.6 94.125) (end 163.825 96.35) (width 0.5) (layer B.Cu) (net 6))
 (segment (start 163.825 102.275) (end 161.65 104.45) (width 0.5) (layer B.Cu) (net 6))
 (segment (start 163.825 96.35) (end 163.825 102.275) (width 0.5) (layer B.Cu) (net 6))
 (segment (start 163.250001 81.974999) (end 161.8 83.425) (width 0.5) (layer B.Cu) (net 6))
 (segment (start 163.250001 74.350001) (end 163.250001 81.974999) (width 0.5) (layer B.Cu) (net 6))
 (segment (start 161.8 72.9) (end 163.250001 74.350001) (width 0.5) (layer B.Cu) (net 6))
 (segment (start 148.9 104.55) (end 142.4 104.55) (width 0.5) (layer F.Cu) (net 7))
 (segment (start 148.9 93.85) (end 142.4 93.85) (width 0.5) (layer F.Cu) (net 7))
 (segment (start 148.9 72.8) (end 142.4 72.8) (width 0.5) (layer F.Cu) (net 7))
 (segment (start 148.9 83.45) (end 142.4 83.45) (width 0.5) (layer F.Cu) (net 7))
 (segment (start 139.725 107.225) (end 142.4 104.55) (width 0.5) (layer F.Cu) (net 7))
 (segment (start 124.975 102.896002) (end 129.303998 107.225) (width 0.5) (layer F.Cu) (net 7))
 (segment (start 115.775 89.875) (end 124.975 99.075) (width 0.5) (layer F.Cu) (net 7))
 (segment (start 129.303998 107.225) (end 139.725 107.225) (width 0.5) (layer F.Cu) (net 7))
 (segment (start 124.975 99.075) (end 124.975 102.896002) (width 0.5) (layer F.Cu) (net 7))
 (segment (start 150.350001 81.999999) (end 148.9 83.45) (width 0.5) (layer B.Cu) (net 7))
 (segment (start 150.350001 74.250001) (end 150.350001 81.999999) (width 0.5) (layer B.Cu) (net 7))
 (segment (start 148.9 72.8) (end 150.350001 74.250001) (width 0.5) (layer B.Cu) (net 7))
 (segment (start 150.350001 92.399999) (end 148.9 93.85) (width 0.5) (layer B.Cu) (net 7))
 (segment (start 150.350001 84.900001) (end 150.350001 92.399999) (width 0.5) (layer B.Cu) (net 7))
 (segment (start 148.9 83.45) (end 150.350001 84.900001) (width 0.5) (layer B.Cu) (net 7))
 (segment (start 150.350001 103.099999) (end 148.9 104.55) (width 0.5) (layer B.Cu) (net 7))
 (segment (start 150.350001 95.300001) (end 150.350001 103.099999) (width 0.5) (layer B.Cu) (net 7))
 (segment (start 148.9 93.85) (end 150.350001 95.300001) (width 0.5) (layer B.Cu) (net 7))
 (segment (start 135.3 104.575) (end 128.8 104.575) (width 0.5) (layer F.Cu) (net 8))
 (segment (start 135.5 93.85) (end 129 93.85) (width 0.5) (layer F.Cu) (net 8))
 (segment (start 135.475 83.475) (end 128.975 83.475) (width 0.5) (layer F.Cu) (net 8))
 (segment (start 135.35 72.725) (end 128.85 72.725) (width 0.5) (layer F.Cu) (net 8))
 (segment (start 117.075001 88.635001) (end 117.135001 88.635001) (width 0.5) (layer F.Cu) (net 8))
 (segment (start 115.775 87.335) (end 117.075001 88.635001) (width 0.5) (layer F.Cu) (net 8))
 (segment (start 117.135001 88.635001) (end 126.2 97.7) (width 0.5) (layer F.Cu) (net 8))
 (segment (start 126.2 101.975) (end 128.8 104.575) (width 0.5) (layer F.Cu) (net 8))
 (segment (start 126.2 97.7) (end 126.2 101.975) (width 0.5) (layer F.Cu) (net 8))
 (segment (start 136.925001 82.024999) (end 135.475 83.475) (width 0.5) (layer B.Cu) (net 8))
 (segment (start 136.925001 74.300001) (end 136.925001 82.024999) (width 0.5) (layer B.Cu) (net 8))
 (segment (start 135.35 72.725) (end 136.925001 74.300001) (width 0.5) (layer B.Cu) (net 8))
 (segment (start 136.950001 84.950001) (end 136.950001 92.399999) (width 0.5) (layer B.Cu) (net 8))
 (segment (start 136.950001 92.399999) (end 135.5 93.85) (width 0.5) (layer B.Cu) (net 8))
 (segment (start 135.475 83.475) (end 136.950001 84.950001) (width 0.5) (layer B.Cu) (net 8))
 (segment (start 136.750001 103.124999) (end 135.3 104.575) (width 0.5) (layer B.Cu) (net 8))
 (segment (start 136.750001 95.100001) (end 136.750001 103.124999) (width 0.5) (layer B.Cu) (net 8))
 (segment (start 135.5 93.85) (end 136.750001 95.100001) (width 0.5) (layer B.Cu) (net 8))
 (segment (start 174.125 100.075) (end 174.2 100) (width 0.5) (layer F.Cu) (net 1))
 (segment (start 128.8 100.075) (end 174.125 100.075) (width 0.5) (layer F.Cu) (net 1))
 (segment (start 128.8 97.82) (end 128.8 100.075) (width 0.5) (layer F.Cu) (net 1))
 (segment (start 115.775 84.795) (end 128.8 97.82) (width 0.5) (layer F.Cu) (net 1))
 (segment (start 174.05 89.35) (end 174.325 89.625) (width 0.5) (layer F.Cu) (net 3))
 (segment (start 129 89.35) (end 174.05 89.35) (width 0.5) (layer F.Cu) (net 3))
 (segment (start 121.905 82.255) (end 129 89.35) (width 0.5) (layer F.Cu) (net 3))
 (segment (start 115.775 82.255) (end 121.905 82.255) (width 0.5) (layer F.Cu) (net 3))
 (segment (start 128.975 78.975) (end 174.325 78.975) (width 0.5) (layer F.Cu) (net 4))
 (segment (start 128.235 79.715) (end 128.975 78.975) (width 0.5) (layer F.Cu) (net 4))
 (segment (start 115.775 79.715) (end 128.235 79.715) (width 0.5) (layer F.Cu) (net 4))
 (segment (start 119.9 77.175) (end 128.85 68.225) (width 0.5) (layer F.Cu) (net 5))
 (segment (start 115.775 77.175) (end 119.9 77.175) (width 0.5) (layer F.Cu) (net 5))
 (segment (start 173.875 68.225) (end 174.225 68.575) (width 0.5) (layer F.Cu) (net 5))
 (segment (start 128.85 68.225) (end 173.875 68.225) (width 0.5) (layer F.Cu) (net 5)))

